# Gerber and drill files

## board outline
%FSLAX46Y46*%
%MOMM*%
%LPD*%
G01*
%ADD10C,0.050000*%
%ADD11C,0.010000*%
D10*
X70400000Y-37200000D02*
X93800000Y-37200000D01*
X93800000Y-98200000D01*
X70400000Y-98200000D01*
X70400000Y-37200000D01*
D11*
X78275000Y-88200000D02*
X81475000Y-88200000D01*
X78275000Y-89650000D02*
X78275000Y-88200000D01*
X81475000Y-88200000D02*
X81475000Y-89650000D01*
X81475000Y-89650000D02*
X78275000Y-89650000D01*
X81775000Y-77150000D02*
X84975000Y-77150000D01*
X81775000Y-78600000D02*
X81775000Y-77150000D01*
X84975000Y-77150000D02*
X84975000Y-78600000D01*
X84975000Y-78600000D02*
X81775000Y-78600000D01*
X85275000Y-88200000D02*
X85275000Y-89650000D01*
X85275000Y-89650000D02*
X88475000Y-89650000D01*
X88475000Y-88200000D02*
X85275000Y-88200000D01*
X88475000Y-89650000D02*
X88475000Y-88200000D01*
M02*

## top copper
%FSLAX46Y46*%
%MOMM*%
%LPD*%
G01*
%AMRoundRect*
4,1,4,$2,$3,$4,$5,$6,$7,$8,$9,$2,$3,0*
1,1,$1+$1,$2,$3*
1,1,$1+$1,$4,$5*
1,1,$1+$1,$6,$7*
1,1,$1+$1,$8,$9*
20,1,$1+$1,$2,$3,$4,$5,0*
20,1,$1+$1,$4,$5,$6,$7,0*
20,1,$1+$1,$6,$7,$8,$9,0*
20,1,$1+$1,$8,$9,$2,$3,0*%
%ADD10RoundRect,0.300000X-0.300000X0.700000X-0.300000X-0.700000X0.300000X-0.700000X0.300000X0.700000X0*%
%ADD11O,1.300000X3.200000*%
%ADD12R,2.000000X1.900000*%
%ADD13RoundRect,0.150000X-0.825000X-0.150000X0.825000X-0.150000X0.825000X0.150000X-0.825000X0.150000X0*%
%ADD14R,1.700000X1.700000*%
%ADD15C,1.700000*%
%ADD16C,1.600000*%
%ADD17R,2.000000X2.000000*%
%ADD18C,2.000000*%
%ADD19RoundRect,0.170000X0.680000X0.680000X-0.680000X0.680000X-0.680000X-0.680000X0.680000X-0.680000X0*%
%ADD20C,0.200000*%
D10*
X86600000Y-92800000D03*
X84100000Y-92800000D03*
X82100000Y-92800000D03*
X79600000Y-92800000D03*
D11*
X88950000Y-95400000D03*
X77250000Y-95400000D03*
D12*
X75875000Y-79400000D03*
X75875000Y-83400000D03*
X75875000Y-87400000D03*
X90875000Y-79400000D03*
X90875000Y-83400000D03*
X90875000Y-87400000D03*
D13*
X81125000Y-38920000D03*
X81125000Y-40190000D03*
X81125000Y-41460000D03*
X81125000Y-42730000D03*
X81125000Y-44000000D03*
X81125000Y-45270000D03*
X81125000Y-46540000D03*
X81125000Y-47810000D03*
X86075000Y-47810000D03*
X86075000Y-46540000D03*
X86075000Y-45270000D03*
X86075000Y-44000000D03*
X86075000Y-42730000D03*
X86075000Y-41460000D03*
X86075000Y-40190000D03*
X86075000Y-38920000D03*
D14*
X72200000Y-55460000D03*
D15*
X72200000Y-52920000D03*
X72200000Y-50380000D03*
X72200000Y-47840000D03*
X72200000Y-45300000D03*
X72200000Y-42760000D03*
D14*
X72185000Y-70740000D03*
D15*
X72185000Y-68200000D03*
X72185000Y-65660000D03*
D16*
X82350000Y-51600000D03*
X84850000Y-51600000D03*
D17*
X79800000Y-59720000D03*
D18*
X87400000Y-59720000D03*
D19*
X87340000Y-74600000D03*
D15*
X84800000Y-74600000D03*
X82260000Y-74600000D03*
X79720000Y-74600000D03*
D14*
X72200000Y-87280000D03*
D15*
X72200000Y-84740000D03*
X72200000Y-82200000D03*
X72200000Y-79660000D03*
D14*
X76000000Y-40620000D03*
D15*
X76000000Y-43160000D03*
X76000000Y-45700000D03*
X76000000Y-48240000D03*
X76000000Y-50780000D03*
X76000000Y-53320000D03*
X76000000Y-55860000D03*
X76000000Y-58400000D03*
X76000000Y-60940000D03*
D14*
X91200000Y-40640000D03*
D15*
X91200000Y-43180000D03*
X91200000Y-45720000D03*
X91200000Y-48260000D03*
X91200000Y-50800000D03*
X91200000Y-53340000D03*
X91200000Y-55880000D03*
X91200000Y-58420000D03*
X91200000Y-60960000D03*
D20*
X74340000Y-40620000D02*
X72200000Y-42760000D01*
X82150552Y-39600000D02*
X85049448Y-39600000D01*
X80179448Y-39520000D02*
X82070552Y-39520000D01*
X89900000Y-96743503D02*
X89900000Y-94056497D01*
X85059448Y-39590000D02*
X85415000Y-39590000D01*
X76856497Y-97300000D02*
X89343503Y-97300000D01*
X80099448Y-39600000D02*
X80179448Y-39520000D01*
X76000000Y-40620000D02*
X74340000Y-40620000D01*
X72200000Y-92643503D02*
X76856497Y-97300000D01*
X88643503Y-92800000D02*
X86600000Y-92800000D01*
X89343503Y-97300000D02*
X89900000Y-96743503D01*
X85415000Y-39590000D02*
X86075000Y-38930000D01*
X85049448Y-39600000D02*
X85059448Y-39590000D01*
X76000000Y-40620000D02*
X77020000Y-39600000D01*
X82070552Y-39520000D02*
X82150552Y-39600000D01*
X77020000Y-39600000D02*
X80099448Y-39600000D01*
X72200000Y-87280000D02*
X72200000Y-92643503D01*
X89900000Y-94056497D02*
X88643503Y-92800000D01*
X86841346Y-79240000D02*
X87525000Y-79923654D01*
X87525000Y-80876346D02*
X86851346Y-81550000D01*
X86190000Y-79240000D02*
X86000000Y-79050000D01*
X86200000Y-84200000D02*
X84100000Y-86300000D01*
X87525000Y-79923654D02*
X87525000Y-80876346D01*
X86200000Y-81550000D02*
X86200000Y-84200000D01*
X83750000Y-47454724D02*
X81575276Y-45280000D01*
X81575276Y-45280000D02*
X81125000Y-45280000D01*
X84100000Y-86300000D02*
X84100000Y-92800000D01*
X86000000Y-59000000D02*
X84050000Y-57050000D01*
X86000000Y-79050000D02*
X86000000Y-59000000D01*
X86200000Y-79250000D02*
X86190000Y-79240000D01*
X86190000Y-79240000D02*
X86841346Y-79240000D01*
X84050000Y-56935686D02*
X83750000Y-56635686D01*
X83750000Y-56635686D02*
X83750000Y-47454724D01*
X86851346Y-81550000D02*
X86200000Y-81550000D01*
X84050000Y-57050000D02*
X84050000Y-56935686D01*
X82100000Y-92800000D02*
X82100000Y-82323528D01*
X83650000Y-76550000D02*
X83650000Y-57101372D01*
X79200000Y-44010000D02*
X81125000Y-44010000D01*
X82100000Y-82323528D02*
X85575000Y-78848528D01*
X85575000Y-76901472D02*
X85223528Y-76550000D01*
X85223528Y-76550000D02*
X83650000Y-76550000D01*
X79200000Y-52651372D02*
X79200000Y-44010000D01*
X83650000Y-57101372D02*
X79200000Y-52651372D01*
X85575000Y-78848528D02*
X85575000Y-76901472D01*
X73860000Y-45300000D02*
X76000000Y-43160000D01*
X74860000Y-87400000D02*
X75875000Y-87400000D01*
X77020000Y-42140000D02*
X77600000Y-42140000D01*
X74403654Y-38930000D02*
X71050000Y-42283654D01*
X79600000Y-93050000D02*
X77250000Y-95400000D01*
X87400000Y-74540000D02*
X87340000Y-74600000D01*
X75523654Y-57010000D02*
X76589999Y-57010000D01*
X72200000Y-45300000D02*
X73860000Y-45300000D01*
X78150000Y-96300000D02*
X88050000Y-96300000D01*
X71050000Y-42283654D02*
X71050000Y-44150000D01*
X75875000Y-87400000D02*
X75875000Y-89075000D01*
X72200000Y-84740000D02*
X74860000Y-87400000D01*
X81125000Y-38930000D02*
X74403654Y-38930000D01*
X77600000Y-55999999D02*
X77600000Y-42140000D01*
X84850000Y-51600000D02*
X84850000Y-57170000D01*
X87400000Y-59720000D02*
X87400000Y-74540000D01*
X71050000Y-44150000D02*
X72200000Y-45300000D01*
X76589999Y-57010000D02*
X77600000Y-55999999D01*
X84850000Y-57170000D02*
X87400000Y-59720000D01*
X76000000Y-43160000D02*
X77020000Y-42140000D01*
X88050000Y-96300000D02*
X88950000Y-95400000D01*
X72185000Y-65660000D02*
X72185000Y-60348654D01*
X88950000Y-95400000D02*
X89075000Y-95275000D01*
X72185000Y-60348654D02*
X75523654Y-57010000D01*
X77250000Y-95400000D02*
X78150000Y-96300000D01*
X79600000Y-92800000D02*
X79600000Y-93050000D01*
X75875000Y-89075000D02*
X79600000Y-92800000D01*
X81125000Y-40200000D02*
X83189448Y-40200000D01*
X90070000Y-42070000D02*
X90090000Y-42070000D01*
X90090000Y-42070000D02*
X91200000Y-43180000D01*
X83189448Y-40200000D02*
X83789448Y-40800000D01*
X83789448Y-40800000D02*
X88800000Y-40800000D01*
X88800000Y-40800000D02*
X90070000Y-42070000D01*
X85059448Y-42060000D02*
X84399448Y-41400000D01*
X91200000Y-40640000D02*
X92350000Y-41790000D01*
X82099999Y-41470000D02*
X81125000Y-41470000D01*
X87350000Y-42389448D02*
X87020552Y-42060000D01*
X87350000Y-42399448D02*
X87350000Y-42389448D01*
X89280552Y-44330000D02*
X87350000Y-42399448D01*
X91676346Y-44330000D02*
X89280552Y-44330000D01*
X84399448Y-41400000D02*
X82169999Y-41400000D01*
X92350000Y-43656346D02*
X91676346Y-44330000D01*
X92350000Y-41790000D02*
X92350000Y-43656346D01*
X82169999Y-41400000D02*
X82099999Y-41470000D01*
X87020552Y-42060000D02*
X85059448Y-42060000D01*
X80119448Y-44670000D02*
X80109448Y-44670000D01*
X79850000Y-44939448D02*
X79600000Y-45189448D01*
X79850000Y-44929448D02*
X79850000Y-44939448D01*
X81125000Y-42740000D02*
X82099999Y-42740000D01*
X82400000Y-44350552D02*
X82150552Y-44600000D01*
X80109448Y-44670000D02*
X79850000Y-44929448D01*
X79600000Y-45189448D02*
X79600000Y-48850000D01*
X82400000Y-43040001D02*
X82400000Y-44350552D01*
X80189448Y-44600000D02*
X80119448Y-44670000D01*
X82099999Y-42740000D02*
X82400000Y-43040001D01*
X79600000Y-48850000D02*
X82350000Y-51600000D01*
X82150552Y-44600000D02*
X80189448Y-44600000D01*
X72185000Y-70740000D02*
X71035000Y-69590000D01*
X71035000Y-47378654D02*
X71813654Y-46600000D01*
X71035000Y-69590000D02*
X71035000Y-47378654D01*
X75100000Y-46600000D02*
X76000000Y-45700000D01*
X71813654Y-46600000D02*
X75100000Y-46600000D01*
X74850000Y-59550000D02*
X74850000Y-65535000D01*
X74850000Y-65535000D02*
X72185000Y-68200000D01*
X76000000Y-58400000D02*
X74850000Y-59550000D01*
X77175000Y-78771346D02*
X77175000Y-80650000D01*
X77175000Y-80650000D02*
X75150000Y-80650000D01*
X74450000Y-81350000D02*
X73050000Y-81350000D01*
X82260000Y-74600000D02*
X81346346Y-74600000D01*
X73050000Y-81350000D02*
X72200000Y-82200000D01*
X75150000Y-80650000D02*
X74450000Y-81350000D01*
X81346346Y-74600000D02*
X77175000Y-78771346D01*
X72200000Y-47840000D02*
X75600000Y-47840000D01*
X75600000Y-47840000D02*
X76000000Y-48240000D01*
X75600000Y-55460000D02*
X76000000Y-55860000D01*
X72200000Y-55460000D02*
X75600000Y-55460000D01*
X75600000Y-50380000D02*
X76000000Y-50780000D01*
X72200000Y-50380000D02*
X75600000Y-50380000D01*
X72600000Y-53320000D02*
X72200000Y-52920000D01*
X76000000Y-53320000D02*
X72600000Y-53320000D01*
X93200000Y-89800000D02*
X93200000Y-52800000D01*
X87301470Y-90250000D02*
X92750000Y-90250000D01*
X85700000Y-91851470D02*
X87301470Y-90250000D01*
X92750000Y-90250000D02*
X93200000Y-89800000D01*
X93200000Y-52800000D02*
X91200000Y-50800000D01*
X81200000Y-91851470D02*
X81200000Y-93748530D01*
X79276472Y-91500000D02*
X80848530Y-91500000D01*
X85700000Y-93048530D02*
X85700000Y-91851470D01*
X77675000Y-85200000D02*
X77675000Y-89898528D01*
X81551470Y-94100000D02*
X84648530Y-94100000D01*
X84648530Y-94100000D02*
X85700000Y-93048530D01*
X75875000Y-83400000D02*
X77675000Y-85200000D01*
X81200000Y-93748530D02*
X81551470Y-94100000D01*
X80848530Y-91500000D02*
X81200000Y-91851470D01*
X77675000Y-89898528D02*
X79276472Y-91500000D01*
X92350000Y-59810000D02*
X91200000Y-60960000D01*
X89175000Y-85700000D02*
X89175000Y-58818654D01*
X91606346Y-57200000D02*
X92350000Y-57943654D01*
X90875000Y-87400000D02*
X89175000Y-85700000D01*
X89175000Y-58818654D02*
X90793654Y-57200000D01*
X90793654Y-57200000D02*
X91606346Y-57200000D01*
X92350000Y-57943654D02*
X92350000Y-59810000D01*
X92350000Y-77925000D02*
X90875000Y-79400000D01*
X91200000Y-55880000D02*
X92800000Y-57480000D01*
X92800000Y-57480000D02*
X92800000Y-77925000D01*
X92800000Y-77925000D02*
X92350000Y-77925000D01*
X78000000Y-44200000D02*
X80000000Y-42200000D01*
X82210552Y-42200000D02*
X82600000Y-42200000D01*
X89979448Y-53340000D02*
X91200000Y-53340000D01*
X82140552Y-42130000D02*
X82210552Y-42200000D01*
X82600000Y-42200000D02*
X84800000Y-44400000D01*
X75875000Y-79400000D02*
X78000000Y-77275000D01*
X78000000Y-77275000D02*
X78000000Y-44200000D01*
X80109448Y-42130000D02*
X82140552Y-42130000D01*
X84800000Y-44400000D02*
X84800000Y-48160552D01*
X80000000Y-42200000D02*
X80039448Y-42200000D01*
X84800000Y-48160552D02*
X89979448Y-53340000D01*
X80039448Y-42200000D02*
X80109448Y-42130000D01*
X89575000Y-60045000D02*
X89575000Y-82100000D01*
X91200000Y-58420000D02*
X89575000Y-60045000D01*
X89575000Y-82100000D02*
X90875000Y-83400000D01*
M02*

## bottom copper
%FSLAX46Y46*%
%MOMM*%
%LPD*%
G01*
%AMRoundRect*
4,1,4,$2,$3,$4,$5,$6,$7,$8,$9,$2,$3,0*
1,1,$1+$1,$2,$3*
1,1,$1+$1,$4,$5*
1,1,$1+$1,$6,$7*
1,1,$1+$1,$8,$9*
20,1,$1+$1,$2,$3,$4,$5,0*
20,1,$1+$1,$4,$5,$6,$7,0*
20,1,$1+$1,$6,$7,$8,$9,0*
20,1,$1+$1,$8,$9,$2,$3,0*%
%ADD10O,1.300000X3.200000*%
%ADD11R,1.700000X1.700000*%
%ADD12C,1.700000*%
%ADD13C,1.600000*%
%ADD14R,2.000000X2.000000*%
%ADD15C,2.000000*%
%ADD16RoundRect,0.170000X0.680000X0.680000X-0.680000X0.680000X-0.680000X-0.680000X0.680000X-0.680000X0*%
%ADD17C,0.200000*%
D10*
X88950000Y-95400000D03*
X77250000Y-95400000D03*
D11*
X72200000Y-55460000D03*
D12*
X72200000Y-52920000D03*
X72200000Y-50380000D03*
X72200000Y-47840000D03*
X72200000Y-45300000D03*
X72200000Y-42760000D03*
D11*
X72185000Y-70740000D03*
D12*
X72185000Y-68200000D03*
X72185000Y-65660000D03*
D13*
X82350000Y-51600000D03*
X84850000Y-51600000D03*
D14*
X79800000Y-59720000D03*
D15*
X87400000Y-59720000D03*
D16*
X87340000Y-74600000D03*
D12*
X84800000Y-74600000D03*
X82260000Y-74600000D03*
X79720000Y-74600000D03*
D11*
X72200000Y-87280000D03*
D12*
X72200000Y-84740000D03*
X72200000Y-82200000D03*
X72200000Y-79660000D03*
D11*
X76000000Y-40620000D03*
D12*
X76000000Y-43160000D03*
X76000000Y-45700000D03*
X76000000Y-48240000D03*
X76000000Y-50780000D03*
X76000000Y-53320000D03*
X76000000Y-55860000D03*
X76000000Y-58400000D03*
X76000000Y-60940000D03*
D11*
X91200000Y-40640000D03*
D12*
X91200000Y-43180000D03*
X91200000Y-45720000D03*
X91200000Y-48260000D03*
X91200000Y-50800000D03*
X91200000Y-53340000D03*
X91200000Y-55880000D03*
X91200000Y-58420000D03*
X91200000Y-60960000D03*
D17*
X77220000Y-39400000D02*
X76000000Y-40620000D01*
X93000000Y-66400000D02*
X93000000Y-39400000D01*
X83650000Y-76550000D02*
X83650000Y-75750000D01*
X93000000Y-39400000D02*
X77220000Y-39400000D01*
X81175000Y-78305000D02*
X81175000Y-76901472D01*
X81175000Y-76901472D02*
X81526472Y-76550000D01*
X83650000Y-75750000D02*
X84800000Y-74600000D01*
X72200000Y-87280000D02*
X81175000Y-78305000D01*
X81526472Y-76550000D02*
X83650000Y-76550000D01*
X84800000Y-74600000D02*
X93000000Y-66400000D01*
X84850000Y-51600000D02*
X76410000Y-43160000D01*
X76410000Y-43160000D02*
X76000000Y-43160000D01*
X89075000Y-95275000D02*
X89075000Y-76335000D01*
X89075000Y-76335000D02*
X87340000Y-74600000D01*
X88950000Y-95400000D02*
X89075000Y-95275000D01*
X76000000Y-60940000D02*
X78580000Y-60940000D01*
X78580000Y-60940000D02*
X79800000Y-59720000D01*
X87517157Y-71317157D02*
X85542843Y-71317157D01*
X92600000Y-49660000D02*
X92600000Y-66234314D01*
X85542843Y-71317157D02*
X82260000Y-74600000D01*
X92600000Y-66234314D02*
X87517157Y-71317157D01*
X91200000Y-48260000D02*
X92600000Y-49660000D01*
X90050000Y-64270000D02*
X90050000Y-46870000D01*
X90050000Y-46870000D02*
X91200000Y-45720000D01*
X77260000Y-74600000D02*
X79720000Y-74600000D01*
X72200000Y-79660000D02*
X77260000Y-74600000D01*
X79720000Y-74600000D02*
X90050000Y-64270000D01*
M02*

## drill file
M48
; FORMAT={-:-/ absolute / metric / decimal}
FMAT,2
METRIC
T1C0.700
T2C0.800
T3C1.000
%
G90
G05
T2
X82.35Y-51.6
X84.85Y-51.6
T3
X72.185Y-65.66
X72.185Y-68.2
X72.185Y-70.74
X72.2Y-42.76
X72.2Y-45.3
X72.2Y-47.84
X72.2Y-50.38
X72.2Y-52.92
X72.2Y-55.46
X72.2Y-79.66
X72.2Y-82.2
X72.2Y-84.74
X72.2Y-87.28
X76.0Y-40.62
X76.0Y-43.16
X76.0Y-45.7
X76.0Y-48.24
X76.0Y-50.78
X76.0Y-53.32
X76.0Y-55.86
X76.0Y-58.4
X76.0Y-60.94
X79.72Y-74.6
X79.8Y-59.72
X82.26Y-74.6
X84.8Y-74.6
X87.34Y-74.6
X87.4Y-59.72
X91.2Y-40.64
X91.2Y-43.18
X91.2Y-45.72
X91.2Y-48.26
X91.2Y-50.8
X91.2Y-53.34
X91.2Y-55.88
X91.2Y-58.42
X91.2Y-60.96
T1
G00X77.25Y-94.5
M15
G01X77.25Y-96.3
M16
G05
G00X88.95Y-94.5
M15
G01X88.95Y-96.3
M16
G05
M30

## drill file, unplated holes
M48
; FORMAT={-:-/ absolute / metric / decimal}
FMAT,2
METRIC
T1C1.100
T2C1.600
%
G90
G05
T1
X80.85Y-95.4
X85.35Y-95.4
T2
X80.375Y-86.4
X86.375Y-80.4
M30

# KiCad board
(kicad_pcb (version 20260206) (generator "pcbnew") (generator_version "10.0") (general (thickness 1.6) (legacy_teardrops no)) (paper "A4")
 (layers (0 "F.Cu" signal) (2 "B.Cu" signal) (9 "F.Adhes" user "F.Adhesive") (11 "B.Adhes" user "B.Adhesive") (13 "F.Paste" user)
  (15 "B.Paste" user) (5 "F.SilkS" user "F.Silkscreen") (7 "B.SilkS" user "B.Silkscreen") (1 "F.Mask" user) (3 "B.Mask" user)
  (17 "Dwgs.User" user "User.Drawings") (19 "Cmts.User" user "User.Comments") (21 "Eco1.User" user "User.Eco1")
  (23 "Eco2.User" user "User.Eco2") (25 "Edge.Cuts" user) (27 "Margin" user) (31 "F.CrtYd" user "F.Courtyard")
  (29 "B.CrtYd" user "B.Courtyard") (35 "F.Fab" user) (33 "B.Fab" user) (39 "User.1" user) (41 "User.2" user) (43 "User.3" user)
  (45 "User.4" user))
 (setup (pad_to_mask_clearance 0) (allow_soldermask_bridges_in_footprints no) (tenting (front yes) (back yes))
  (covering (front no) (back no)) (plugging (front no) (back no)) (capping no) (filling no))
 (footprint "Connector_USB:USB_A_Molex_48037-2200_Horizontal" (layer "F.Cu") (at 83.1 103.775 -90)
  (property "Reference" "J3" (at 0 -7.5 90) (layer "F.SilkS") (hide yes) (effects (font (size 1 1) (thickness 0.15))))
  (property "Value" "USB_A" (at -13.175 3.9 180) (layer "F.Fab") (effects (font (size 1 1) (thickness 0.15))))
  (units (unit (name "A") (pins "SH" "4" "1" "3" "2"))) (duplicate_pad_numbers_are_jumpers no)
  (pad "" np_thru_hole circle (at -8.375 -2.25 270) (size 1.1 1.1) (drill 1.1) (layers "*.Mask"))
  (pad "" np_thru_hole circle (at -8.375 2.25 270) (size 1.1 1.1) (drill 1.1) (layers "*.Mask"))
  (pad "1" smd roundrect (at -10.975 -3.5 270) (size 2 1.2) (layers "F.Cu" "F.Mask" "F.Paste") (roundrect_rratio 0.25) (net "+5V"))
  (pad "2" smd roundrect (at -10.975 -1 270) (size 2 1.2) (layers "F.Cu" "F.Mask" "F.Paste") (roundrect_rratio 0.25) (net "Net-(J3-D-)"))
  (pad "3" smd roundrect (at -10.975 1 270) (size 2 1.2) (layers "F.Cu" "F.Mask" "F.Paste") (roundrect_rratio 0.25) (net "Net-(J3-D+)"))
  (pad "4" smd roundrect (at -10.975 3.5 270) (size 2 1.2) (layers "F.Cu" "F.Mask" "F.Paste") (roundrect_rratio 0.25) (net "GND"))
  (pad "SH" thru_hole oval (at -8.375 -5.85 270) (size 3.2 1.3) (drill oval 2.5 0.7) (layers "*.Cu" "*.Mask") (remove_unused_layers no)
   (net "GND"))
  (pad "SH" thru_hole oval (at -8.375 5.85 270) (size 3.2 1.3) (drill oval 2.5 0.7) (layers "*.Cu" "*.Mask") (remove_unused_layers no)
   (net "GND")))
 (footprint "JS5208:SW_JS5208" (layer "F.Cu") (at 83.375 83.4)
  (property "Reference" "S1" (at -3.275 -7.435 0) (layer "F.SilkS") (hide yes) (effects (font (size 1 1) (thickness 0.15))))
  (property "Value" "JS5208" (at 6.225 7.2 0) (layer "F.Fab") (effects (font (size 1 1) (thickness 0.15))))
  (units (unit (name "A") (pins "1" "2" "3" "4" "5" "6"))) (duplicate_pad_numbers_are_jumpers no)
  (fp_line (start -5.1 4.8) (end -1.9 4.8) (stroke (width 0.01) (type solid)) (layer "Edge.Cuts"))
  (fp_line (start -5.1 6.25) (end -5.1 4.8) (stroke (width 0.01) (type solid)) (layer "Edge.Cuts"))
  (fp_line (start -1.9 4.8) (end -1.9 6.25) (stroke (width 0.01) (type solid)) (layer "Edge.Cuts"))
  (fp_line (start -1.9 6.25) (end -5.1 6.25) (stroke (width 0.01) (type solid)) (layer "Edge.Cuts"))
  (fp_line (start -1.6 -6.25) (end 1.6 -6.25) (stroke (width 0.01) (type solid)) (layer "Edge.Cuts"))
  (fp_line (start -1.6 -4.8) (end -1.6 -6.25) (stroke (width 0.01) (type solid)) (layer "Edge.Cuts"))
  (fp_line (start 1.6 -6.25) (end 1.6 -4.8) (stroke (width 0.01) (type solid)) (layer "Edge.Cuts"))
  (fp_line (start 1.6 -4.8) (end -1.6 -4.8) (stroke (width 0.01) (type solid)) (layer "Edge.Cuts"))
  (fp_line (start 1.9 4.8) (end 1.9 6.25) (stroke (width 0.01) (type solid)) (layer "Edge.Cuts"))
  (fp_line (start 1.9 6.25) (end 5.1 6.25) (stroke (width 0.01) (type solid)) (layer "Edge.Cuts"))
  (fp_line (start 5.1 4.8) (end 1.9 4.8) (stroke (width 0.01) (type solid)) (layer "Edge.Cuts"))
  (fp_line (start 5.1 6.25) (end 5.1 4.8) (stroke (width 0.01) (type solid)) (layer "Edge.Cuts"))
  (pad "" np_thru_hole circle (at -3 3) (size 1.6 1.6) (drill 1.6) (layers "*.Cu" "*.Mask"))
  (pad "" np_thru_hole circle (at 3 -3) (size 1.6 1.6) (drill 1.6) (layers "*.Cu" "*.Mask"))
  (pad "1" smd rect (at -7.5 -4) (size 2 1.9) (layers "F.Cu" "F.Mask" "F.Paste") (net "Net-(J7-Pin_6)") (solder_mask_margin 0.102))
  (pad "2" smd rect (at -7.5 0) (size 2 1.9) (layers "F.Cu" "F.Mask" "F.Paste") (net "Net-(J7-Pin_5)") (solder_mask_margin 0.102))
  (pad "3" smd rect (at -7.5 4) (size 2 1.9) (layers "F.Cu" "F.Mask" "F.Paste") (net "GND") (solder_mask_margin 0.102))
  (pad "4" smd rect (at 7.5 -4) (size 2 1.9) (layers "F.Cu" "F.Mask" "F.Paste") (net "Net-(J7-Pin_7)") (solder_mask_margin 0.102))
  (pad "5" smd rect (at 7.5 0) (size 2 1.9) (layers "F.Cu" "F.Mask" "F.Paste") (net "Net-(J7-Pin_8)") (solder_mask_margin 0.102))
  (pad "6" smd rect (at 7.5 4) (size 2 1.9) (layers "F.Cu" "F.Mask" "F.Paste") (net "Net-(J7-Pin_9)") (solder_mask_margin 0.102)))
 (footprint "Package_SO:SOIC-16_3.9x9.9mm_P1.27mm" (layer "F.Cu") (at 83.6 43.365)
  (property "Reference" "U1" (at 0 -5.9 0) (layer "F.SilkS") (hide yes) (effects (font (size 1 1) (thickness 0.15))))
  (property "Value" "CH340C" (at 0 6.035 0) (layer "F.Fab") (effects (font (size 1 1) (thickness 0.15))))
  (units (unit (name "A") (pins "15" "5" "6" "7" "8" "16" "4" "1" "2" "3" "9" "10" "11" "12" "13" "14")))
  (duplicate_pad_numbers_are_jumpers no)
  (pad "1" smd roundrect (at -2.475 -4.445) (size 1.95 0.6) (layers "F.Cu" "F.Mask" "F.Paste") (roundrect_rratio 0.25) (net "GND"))
  (pad "2" smd roundrect (at -2.475 -3.175) (size 1.95 0.6) (layers "F.Cu" "F.Mask" "F.Paste") (roundrect_rratio 0.25)
   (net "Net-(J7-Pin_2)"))
  (pad "3" smd roundrect (at -2.475 -1.905) (size 1.95 0.6) (layers "F.Cu" "F.Mask" "F.Paste") (roundrect_rratio 0.25)
   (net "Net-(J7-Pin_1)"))
  (pad "4" smd roundrect (at -2.475 -0.635) (size 1.95 0.6) (layers "F.Cu" "F.Mask" "F.Paste") (roundrect_rratio 0.25) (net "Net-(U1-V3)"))
  (pad "5" smd roundrect (at -2.475 0.635) (size 1.95 0.6) (layers "F.Cu" "F.Mask" "F.Paste") (roundrect_rratio 0.25) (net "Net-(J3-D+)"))
  (pad "6" smd roundrect (at -2.475 1.905) (size 1.95 0.6) (layers "F.Cu" "F.Mask" "F.Paste") (roundrect_rratio 0.25) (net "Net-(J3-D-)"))
  (pad "7" smd roundrect (at -2.475 3.175) (size 1.95 0.6) (layers "F.Cu" "F.Mask" "F.Paste") (roundrect_rratio 0.25)
   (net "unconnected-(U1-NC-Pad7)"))
  (pad "8" smd roundrect (at -2.475 4.445) (size 1.95 0.6) (layers "F.Cu" "F.Mask" "F.Paste") (roundrect_rratio 0.25)
   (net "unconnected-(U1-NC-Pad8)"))
  (pad "9" smd roundrect (at 2.475 4.445) (size 1.95 0.6) (layers "F.Cu" "F.Mask" "F.Paste") (roundrect_rratio 0.25)
   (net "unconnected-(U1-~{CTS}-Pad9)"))
  (pad "10" smd roundrect (at 2.475 3.175) (size 1.95 0.6) (layers "F.Cu" "F.Mask" "F.Paste") (roundrect_rratio 0.25)
   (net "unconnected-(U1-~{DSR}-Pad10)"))
  (pad "11" smd roundrect (at 2.475 1.905) (size 1.95 0.6) (layers "F.Cu" "F.Mask" "F.Paste") (roundrect_rratio 0.25)
   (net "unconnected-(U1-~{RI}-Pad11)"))
  (pad "12" smd roundrect (at 2.475 0.635) (size 1.95 0.6) (layers "F.Cu" "F.Mask" "F.Paste") (roundrect_rratio 0.25)
   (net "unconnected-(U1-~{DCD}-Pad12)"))
  (pad "13" smd roundrect (at 2.475 -0.635) (size 1.95 0.6) (layers "F.Cu" "F.Mask" "F.Paste") (roundrect_rratio 0.25)
   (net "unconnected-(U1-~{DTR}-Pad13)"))
  (pad "14" smd roundrect (at 2.475 -1.905) (size 1.95 0.6) (layers "F.Cu" "F.Mask" "F.Paste") (roundrect_rratio 0.25)
   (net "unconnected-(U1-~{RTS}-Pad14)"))
  (pad "15" smd roundrect (at 2.475 -3.175) (size 1.95 0.6) (layers "F.Cu" "F.Mask" "F.Paste") (roundrect_rratio 0.25)
   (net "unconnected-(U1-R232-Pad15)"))
  (pad "16" smd roundrect (at 2.475 -4.445) (size 1.95 0.6) (layers "F.Cu" "F.Mask" "F.Paste") (roundrect_rratio 0.25) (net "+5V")))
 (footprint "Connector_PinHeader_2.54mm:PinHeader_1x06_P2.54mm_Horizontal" (layer "F.Cu") (at 72.2 55.46 180)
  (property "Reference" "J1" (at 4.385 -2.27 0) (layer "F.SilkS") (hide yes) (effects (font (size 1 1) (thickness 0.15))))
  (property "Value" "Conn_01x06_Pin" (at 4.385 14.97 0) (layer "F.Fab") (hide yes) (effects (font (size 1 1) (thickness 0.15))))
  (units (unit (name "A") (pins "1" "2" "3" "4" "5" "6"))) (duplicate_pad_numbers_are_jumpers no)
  (pad "1" thru_hole rect (at 0 0 180) (size 1.7 1.7) (drill 1) (layers "*.Cu" "*.Mask") (remove_unused_layers no) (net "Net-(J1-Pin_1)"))
  (pad "2" thru_hole circle (at 0 2.54 180) (size 1.7 1.7) (drill 1) (layers "*.Cu" "*.Mask") (remove_unused_layers no)
   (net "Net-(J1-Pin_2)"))
  (pad "3" thru_hole circle (at 0 5.08 180) (size 1.7 1.7) (drill 1) (layers "*.Cu" "*.Mask") (remove_unused_layers no)
   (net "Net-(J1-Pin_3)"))
  (pad "4" thru_hole circle (at 0 7.62 180) (size 1.7 1.7) (drill 1) (layers "*.Cu" "*.Mask") (remove_unused_layers no)
   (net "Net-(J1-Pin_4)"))
  (pad "5" thru_hole circle (at 0 10.16 180) (size 1.7 1.7) (drill 1) (layers "*.Cu" "*.Mask") (remove_unused_layers no) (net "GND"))
  (pad "6" thru_hole circle (at 0 12.7 180) (size 1.7 1.7) (drill 1) (layers "*.Cu" "*.Mask") (remove_unused_layers no) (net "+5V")))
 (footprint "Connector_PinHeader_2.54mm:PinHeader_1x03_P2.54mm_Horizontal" (layer "F.Cu") (at 72.185 70.74 180)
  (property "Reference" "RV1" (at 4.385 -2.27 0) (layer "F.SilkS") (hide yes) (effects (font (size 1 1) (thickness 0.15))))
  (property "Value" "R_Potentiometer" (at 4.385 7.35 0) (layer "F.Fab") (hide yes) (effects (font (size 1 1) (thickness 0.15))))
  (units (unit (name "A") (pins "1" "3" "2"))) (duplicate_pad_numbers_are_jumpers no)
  (pad "1" thru_hole rect (at 0 0 180) (size 1.7 1.7) (drill 1) (layers "*.Cu" "*.Mask") (remove_unused_layers no) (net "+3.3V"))
  (pad "2" thru_hole circle (at 0 2.54 180) (size 1.7 1.7) (drill 1) (layers "*.Cu" "*.Mask") (remove_unused_layers no) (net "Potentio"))
  (pad "3" thru_hole circle (at 0 5.08 180) (size 1.7 1.7) (drill 1) (layers "*.Cu" "*.Mask") (remove_unused_layers no) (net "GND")))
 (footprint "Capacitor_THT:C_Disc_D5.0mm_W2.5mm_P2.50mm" (layer "F.Cu") (at 82.35 51.6)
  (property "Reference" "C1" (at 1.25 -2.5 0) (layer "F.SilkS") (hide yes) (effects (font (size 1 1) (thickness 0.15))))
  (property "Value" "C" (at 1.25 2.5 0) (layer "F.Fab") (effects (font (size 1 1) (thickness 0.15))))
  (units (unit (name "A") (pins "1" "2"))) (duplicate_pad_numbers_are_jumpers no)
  (pad "1" thru_hole circle (at 0 0) (size 1.6 1.6) (drill 0.8) (layers "*.Cu" "*.Mask") (remove_unused_layers no) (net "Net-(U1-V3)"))
  (pad "2" thru_hole circle (at 2.5 0) (size 1.6 1.6) (drill 0.8) (layers "*.Cu" "*.Mask") (remove_unused_layers no) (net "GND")))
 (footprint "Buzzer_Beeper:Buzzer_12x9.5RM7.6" (layer "F.Cu") (at 79.8 59.72)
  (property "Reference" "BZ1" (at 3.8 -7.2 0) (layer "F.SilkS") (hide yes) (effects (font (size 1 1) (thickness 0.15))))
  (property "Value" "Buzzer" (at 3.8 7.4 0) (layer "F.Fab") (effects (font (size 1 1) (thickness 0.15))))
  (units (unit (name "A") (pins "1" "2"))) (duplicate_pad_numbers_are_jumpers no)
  (pad "1" thru_hole rect (at 0 0) (size 2 2) (drill 1) (layers "*.Cu" "*.Mask") (remove_unused_layers no) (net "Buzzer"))
  (pad "2" thru_hole circle (at 7.6 0) (size 2 2) (drill 1) (layers "*.Cu" "*.Mask") (remove_unused_layers no) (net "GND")))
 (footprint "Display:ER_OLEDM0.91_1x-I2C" (layer "F.Cu") (at 87.34 74.6 180)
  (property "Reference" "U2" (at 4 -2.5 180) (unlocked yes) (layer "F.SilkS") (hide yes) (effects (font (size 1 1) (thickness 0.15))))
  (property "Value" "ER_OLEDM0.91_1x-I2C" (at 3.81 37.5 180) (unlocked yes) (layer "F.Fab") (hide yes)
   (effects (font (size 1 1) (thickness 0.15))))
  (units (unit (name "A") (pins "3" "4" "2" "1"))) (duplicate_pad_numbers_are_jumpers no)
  (pad "1" thru_hole roundrect (at 0 0 180) (size 1.7 1.7) (drill 1) (layers "*.Cu" "*.Mask") (remove_unused_layers no)
   (roundrect_rratio 0.1) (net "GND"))
  (pad "2" thru_hole circle (at 2.54 0 180) (size 1.7 1.7) (drill 1) (layers "*.Cu" "*.Mask") (remove_unused_layers no) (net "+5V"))
  (pad "3" thru_hole circle (at 5.08 0 180) (size 1.7 1.7) (drill 1) (layers "*.Cu" "*.Mask") (remove_unused_layers no) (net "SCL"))
  (pad "4" thru_hole circle (at 7.62 0 180) (size 1.7 1.7) (drill 1) (layers "*.Cu" "*.Mask") (remove_unused_layers no) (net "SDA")))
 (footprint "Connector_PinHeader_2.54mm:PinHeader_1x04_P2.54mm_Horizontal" (layer "F.Cu") (at 72.2 87.28 180)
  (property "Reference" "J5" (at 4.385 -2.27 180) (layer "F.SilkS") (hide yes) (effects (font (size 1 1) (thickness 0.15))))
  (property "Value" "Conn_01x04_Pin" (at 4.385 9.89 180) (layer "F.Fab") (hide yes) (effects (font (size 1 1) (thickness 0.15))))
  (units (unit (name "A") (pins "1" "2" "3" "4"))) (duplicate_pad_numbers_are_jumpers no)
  (pad "1" thru_hole rect (at 0 0 180) (size 1.7 1.7) (drill 1) (layers "*.Cu" "*.Mask") (remove_unused_layers no) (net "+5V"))
  (pad "2" thru_hole circle (at 0 2.54 180) (size 1.7 1.7) (drill 1) (layers "*.Cu" "*.Mask") (remove_unused_layers no) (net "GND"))
  (pad "3" thru_hole circle (at 0 5.08 180) (size 1.7 1.7) (drill 1) (layers "*.Cu" "*.Mask") (remove_unused_layers no) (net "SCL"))
  (pad "4" thru_hole circle (at 0 7.62 180) (size 1.7 1.7) (drill 1) (layers "*.Cu" "*.Mask") (remove_unused_layers no) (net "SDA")))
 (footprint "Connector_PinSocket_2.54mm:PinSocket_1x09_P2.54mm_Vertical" (layer "B.Cu") (at 76 40.62 180)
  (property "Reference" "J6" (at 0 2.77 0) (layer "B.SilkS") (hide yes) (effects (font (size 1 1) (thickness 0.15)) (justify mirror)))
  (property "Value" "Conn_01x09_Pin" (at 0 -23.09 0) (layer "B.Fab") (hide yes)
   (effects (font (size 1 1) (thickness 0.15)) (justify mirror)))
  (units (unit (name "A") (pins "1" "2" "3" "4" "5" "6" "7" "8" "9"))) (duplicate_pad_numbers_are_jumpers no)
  (pad "1" thru_hole rect (at 0 0 180) (size 1.7 1.7) (drill 1) (layers "*.Cu" "*.Mask") (remove_unused_layers no) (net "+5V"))
  (pad "2" thru_hole circle (at 0 -2.54 180) (size 1.7 1.7) (drill 1) (layers "*.Cu" "*.Mask") (remove_unused_layers no) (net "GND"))
  (pad "3" thru_hole circle (at 0 -5.08 180) (size 1.7 1.7) (drill 1) (layers "*.Cu" "*.Mask") (remove_unused_layers no) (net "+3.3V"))
  (pad "4" thru_hole circle (at 0 -7.62 180) (size 1.7 1.7) (drill 1) (layers "*.Cu" "*.Mask") (remove_unused_layers no)
   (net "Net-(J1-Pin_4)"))
  (pad "5" thru_hole circle (at 0 -10.16 180) (size 1.7 1.7) (drill 1) (layers "*.Cu" "*.Mask") (remove_unused_layers no)
   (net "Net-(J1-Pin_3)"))
  (pad "6" thru_hole circle (at 0 -12.7 180) (size 1.7 1.7) (drill 1) (layers "*.Cu" "*.Mask") (remove_unused_layers no)
   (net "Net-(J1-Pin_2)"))
  (pad "7" thru_hole circle (at 0 -15.24 180) (size 1.7 1.7) (drill 1) (layers "*.Cu" "*.Mask") (remove_unused_layers no)
   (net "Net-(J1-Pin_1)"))
  (pad "8" thru_hole circle (at 0 -17.78 180) (size 1.7 1.7) (drill 1) (layers "*.Cu" "*.Mask") (remove_unused_layers no) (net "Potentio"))
  (pad "9" thru_hole circle (at 0 -20.32 180) (size 1.7 1.7) (drill 1) (layers "*.Cu" "*.Mask") (remove_unused_layers no) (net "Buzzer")))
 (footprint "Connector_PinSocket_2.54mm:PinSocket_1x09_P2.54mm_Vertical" (layer "B.Cu") (at 91.2 40.64 180)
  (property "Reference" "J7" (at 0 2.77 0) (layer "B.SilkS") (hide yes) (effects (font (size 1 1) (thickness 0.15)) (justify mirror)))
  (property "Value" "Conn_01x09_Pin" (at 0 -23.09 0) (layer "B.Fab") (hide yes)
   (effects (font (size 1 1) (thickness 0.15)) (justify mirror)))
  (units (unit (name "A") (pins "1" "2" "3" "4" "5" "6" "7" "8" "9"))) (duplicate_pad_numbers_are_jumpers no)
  (pad "1" thru_hole rect (at 0 0 180) (size 1.7 1.7) (drill 1) (layers "*.Cu" "*.Mask") (remove_unused_layers no) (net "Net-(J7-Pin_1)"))
  (pad "2" thru_hole circle (at 0 -2.54 180) (size 1.7 1.7) (drill 1) (layers "*.Cu" "*.Mask") (remove_unused_layers no)
   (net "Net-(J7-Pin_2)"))
  (pad "3" thru_hole circle (at 0 -5.08 180) (size 1.7 1.7) (drill 1) (layers "*.Cu" "*.Mask") (remove_unused_layers no) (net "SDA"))
  (pad "4" thru_hole circle (at 0 -7.62 180) (size 1.7 1.7) (drill 1) (layers "*.Cu" "*.Mask") (remove_unused_layers no) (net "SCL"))
  (pad "5" thru_hole circle (at 0 -10.16 180) (size 1.7 1.7) (drill 1) (layers "*.Cu" "*.Mask") (remove_unused_layers no)
   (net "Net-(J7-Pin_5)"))
  (pad "6" thru_hole circle (at 0 -12.7 180) (size 1.7 1.7) (drill 1) (layers "*.Cu" "*.Mask") (remove_unused_layers no)
   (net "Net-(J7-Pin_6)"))
  (pad "7" thru_hole circle (at 0 -15.24 180) (size 1.7 1.7) (drill 1) (layers "*.Cu" "*.Mask") (remove_unused_layers no)
   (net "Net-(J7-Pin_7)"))
  (pad "8" thru_hole circle (at 0 -17.78 180) (size 1.7 1.7) (drill 1) (layers "*.Cu" "*.Mask") (remove_unused_layers no)
   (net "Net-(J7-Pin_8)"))
  (pad "9" thru_hole circle (at 0 -20.32 180) (size 1.7 1.7) (drill 1) (layers "*.Cu" "*.Mask") (remove_unused_layers no)
   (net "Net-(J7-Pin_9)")))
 (gr_rect (start 70.4 37.2) (end 93.8 98.2) (stroke (width 0.05) (type default)) (fill no) (layer "Edge.Cuts"))
 (segment (start 74.34 40.62) (end 72.2 42.76) (width 0.2) (layer "F.Cu") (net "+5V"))
 (segment (start 82.150552 39.6) (end 85.049448 39.6) (width 0.2) (layer "F.Cu") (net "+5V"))
 (segment (start 80.179448 39.52) (end 82.070552 39.52) (width 0.2) (layer "F.Cu") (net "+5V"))
 (segment (start 89.9 96.743503) (end 89.9 94.056497) (width 0.2) (layer "F.Cu") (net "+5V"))
 (segment (start 85.059448 39.59) (end 85.415 39.59) (width 0.2) (layer "F.Cu") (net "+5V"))
 (segment (start 76.856497 97.3) (end 89.343503 97.3) (width 0.2) (layer "F.Cu") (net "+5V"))
 (segment (start 80.099448 39.6) (end 80.179448 39.52) (width 0.2) (layer "F.Cu") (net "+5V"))
 (segment (start 76 40.62) (end 74.34 40.62) (width 0.2) (layer "F.Cu") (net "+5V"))
 (segment (start 72.2 92.643503) (end 76.856497 97.3) (width 0.2) (layer "F.Cu") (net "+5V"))
 (segment (start 88.643503 92.8) (end 86.6 92.8) (width 0.2) (layer "F.Cu") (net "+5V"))
 (segment (start 89.343503 97.3) (end 89.9 96.743503) (width 0.2) (layer "F.Cu") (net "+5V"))
 (segment (start 85.415 39.59) (end 86.075 38.93) (width 0.2) (layer "F.Cu") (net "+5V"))
 (segment (start 85.049448 39.6) (end 85.059448 39.59) (width 0.2) (layer "F.Cu") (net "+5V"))
 (segment (start 76 40.62) (end 77.02 39.6) (width 0.2) (layer "F.Cu") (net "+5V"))
 (segment (start 82.070552 39.52) (end 82.150552 39.6) (width 0.2) (layer "F.Cu") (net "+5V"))
 (segment (start 77.02 39.6) (end 80.099448 39.6) (width 0.2) (layer "F.Cu") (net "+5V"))
 (segment (start 72.2 87.28) (end 72.2 92.643503) (width 0.2) (layer "F.Cu") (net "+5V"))
 (segment (start 89.9 94.056497) (end 88.643503 92.8) (width 0.2) (layer "F.Cu") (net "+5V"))
 (segment (start 77.22 39.4) (end 76 40.62) (width 0.2) (layer "B.Cu") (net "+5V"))
 (segment (start 93 66.4) (end 93 39.4) (width 0.2) (layer "B.Cu") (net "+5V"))
 (segment (start 83.65 76.55) (end 83.65 75.75) (width 0.2) (layer "B.Cu") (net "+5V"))
 (segment (start 93 39.4) (end 77.22 39.4) (width 0.2) (layer "B.Cu") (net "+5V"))
 (segment (start 81.175 78.305) (end 81.175 76.901472) (width 0.2) (layer "B.Cu") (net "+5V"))
 (segment (start 81.175 76.901472) (end 81.526472 76.55) (width 0.2) (layer "B.Cu") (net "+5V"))
 (segment (start 83.65 75.75) (end 84.8 74.6) (width 0.2) (layer "B.Cu") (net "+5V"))
 (segment (start 72.2 87.28) (end 81.175 78.305) (width 0.2) (layer "B.Cu") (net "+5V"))
 (segment (start 81.526472 76.55) (end 83.65 76.55) (width 0.2) (layer "B.Cu") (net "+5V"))
 (segment (start 84.8 74.6) (end 93 66.4) (width 0.2) (layer "B.Cu") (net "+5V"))
 (segment (start 86.841346 79.24) (end 87.525 79.923654) (width 0.2) (layer "F.Cu") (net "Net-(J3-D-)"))
 (segment (start 87.525 80.876346) (end 86.851346 81.55) (width 0.2) (layer "F.Cu") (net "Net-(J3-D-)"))
 (segment (start 86.19 79.24) (end 86 79.05) (width 0.2) (layer "F.Cu") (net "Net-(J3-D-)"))
 (segment (start 86.2 84.2) (end 84.1 86.3) (width 0.2) (layer "F.Cu") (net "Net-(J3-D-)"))
 (segment (start 87.525 79.923654) (end 87.525 80.876346) (width 0.2) (layer "F.Cu") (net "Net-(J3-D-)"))
 (segment (start 86.2 81.55) (end 86.2 84.2) (width 0.2) (layer "F.Cu") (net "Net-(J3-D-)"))
 (segment (start 83.75 47.454724) (end 81.575276 45.28) (width 0.2) (layer "F.Cu") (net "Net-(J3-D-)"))
 (segment (start 81.575276 45.28) (end 81.125 45.28) (width 0.2) (layer "F.Cu") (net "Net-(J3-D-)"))
 (segment (start 84.1 86.3) (end 84.1 92.8) (width 0.2) (layer "F.Cu") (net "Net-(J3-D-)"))
 (segment (start 86 59) (end 84.05 57.05) (width 0.2) (layer "F.Cu") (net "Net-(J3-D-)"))
 (segment (start 86 79.05) (end 86 59) (width 0.2) (layer "F.Cu") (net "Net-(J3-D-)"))
 (segment (start 86.2 79.25) (end 86.19 79.24) (width 0.2) (layer "F.Cu") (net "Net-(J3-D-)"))
 (segment (start 86.19 79.24) (end 86.841346 79.24) (width 0.2) (layer "F.Cu") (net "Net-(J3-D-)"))
 (segment (start 84.05 56.935686) (end 83.75 56.635686) (width 0.2) (layer "F.Cu") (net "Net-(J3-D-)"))
 (segment (start 83.75 56.635686) (end 83.75 47.454724) (width 0.2) (layer "F.Cu") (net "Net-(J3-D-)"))
 (segment (start 86.851346 81.55) (end 86.2 81.55) (width 0.2) (layer "F.Cu") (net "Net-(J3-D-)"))
 (segment (start 84.05 57.05) (end 84.05 56.935686) (width 0.2) (layer "F.Cu") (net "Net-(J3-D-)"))
 (segment (start 82.1 92.8) (end 82.1 82.323528) (width 0.2) (layer "F.Cu") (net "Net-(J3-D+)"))
 (segment (start 83.65 76.55) (end 83.65 57.101372) (width 0.2) (layer "F.Cu") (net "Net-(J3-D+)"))
 (segment (start 79.2 44.01) (end 81.125 44.01) (width 0.2) (layer "F.Cu") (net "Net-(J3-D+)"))
 (segment (start 82.1 82.323528) (end 85.575 78.848528) (width 0.2) (layer "F.Cu") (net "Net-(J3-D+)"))
 (segment (start 85.575 76.901472) (end 85.223528 76.55) (width 0.2) (layer "F.Cu") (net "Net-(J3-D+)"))
 (segment (start 85.223528 76.55) (end 83.65 76.55) (width 0.2) (layer "F.Cu") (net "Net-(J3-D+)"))
 (segment (start 79.2 52.651372) (end 79.2 44.01) (width 0.2) (layer "F.Cu") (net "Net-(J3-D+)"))
 (segment (start 83.65 57.101372) (end 79.2 52.651372) (width 0.2) (layer "F.Cu") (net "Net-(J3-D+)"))
 (segment (start 85.575 78.848528) (end 85.575 76.901472) (width 0.2) (layer "F.Cu") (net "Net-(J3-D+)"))
 (segment (start 73.86 45.3) (end 76 43.16) (width 0.2) (layer "F.Cu") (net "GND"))
 (segment (start 74.86 87.4) (end 75.875 87.4) (width 0.2) (layer "F.Cu") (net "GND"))
 (segment (start 77.02 42.14) (end 77.6 42.14) (width 0.2) (layer "F.Cu") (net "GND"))
 (segment (start 74.403654 38.93) (end 71.05 42.283654) (width 0.2) (layer "F.Cu") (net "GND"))
 (segment (start 79.6 93.05) (end 77.25 95.4) (width 0.2) (layer "F.Cu") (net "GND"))
 (segment (start 87.4 74.54) (end 87.34 74.6) (width 0.2) (layer "F.Cu") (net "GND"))
 (segment (start 75.523654 57.01) (end 76.589999 57.01) (width 0.2) (layer "F.Cu") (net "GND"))
 (segment (start 72.2 45.3) (end 73.86 45.3) (width 0.2) (layer "F.Cu") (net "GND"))
 (segment (start 78.15 96.3) (end 88.05 96.3) (width 0.2) (layer "F.Cu") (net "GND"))
 (segment (start 71.05 42.283654) (end 71.05 44.15) (width 0.2) (layer "F.Cu") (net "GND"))
 (segment (start 75.875 87.4) (end 75.875 89.075) (width 0.2) (layer "F.Cu") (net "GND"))
 (segment (start 72.2 84.74) (end 74.86 87.4) (width 0.2) (layer "F.Cu") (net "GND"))
 (segment (start 81.125 38.93) (end 74.403654 38.93) (width 0.2) (layer "F.Cu") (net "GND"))
 (segment (start 77.6 55.999999) (end 77.6 42.14) (width 0.2) (layer "F.Cu") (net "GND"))
 (segment (start 84.85 51.6) (end 84.85 57.17) (width 0.2) (layer "F.Cu") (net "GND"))
 (segment (start 87.4 59.72) (end 87.4 74.54) (width 0.2) (layer "F.Cu") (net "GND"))
 (segment (start 71.05 44.15) (end 72.2 45.3) (width 0.2) (layer "F.Cu") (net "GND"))
 (segment (start 76.589999 57.01) (end 77.6 55.999999) (width 0.2) (layer "F.Cu") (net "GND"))
 (segment (start 84.85 57.17) (end 87.4 59.72) (width 0.2) (layer "F.Cu") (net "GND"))
 (segment (start 76 43.16) (end 77.02 42.14) (width 0.2) (layer "F.Cu") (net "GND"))
 (segment (start 88.05 96.3) (end 88.95 95.4) (width 0.2) (layer "F.Cu") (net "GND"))
 (segment (start 72.185 65.66) (end 72.185 60.348654) (width 0.2) (layer "F.Cu") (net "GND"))
 (segment (start 88.95 95.4) (end 89.075 95.275) (width 0.2) (layer "F.Cu") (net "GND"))
 (segment (start 72.185 60.348654) (end 75.523654 57.01) (width 0.2) (layer "F.Cu") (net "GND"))
 (segment (start 77.25 95.4) (end 78.15 96.3) (width 0.2) (layer "F.Cu") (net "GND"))
 (segment (start 79.6 92.8) (end 79.6 93.05) (width 0.2) (layer "F.Cu") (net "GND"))
 (segment (start 75.875 89.075) (end 79.6 92.8) (width 0.2) (layer "F.Cu") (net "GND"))
 (segment (start 84.85 51.6) (end 76.41 43.16) (width 0.2) (layer "B.Cu") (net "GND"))
 (segment (start 76.41 43.16) (end 76 43.16) (width 0.2) (layer "B.Cu") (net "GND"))
 (segment (start 89.075 95.275) (end 89.075 76.335) (width 0.2) (layer "B.Cu") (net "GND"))
 (segment (start 89.075 76.335) (end 87.34 74.6) (width 0.2) (layer "B.Cu") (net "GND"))
 (segment (start 88.95 95.4) (end 89.075 95.275) (width 0.2) (layer "B.Cu") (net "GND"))
 (segment (start 78 44.2) (end 80 42.2) (width 0.2) (layer "F.Cu") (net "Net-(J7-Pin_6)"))
 (segment (start 82.210552 42.2) (end 82.6 42.2) (width 0.2) (layer "F.Cu") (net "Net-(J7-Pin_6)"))
 (segment (start 89.979448 53.34) (end 91.2 53.34) (width 0.2) (layer "F.Cu") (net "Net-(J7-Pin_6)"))
 (segment (start 82.140552 42.13) (end 82.210552 42.2) (width 0.2) (layer "F.Cu") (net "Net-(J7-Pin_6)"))
 (segment (start 82.6 42.2) (end 84.8 44.4) (width 0.2) (layer "F.Cu") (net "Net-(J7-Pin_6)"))
 (segment (start 75.875 79.4) (end 78 77.275) (width 0.2) (layer "F.Cu") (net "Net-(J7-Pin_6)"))
 (segment (start 78 77.275) (end 78 44.2) (width 0.2) (layer "F.Cu") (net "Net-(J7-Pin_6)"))
 (segment (start 80.109448 42.13) (end 82.140552 42.13) (width 0.2) (layer "F.Cu") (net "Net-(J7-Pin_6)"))
 (segment (start 84.8 44.4) (end 84.8 48.160552) (width 0.2) (layer "F.Cu") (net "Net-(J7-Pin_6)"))
 (segment (start 80 42.2) (end 80.039448 42.2) (width 0.2) (layer "F.Cu") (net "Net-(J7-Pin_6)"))
 (segment (start 84.8 48.160552) (end 89.979448 53.34) (width 0.2) (layer "F.Cu") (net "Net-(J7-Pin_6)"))
 (segment (start 80.039448 42.2) (end 80.109448 42.13) (width 0.2) (layer "F.Cu") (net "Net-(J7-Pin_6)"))
 (segment (start 93.2 89.8) (end 93.2 52.8) (width 0.2) (layer "F.Cu") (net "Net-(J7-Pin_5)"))
 (segment (start 87.30147 90.25) (end 92.75 90.25) (width 0.2) (layer "F.Cu") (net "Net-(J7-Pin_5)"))
 (segment (start 85.7 91.85147) (end 87.30147 90.25) (width 0.2) (layer "F.Cu") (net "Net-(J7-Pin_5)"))
 (segment (start 92.75 90.25) (end 93.2 89.8) (width 0.2) (layer "F.Cu") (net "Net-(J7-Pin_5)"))
 (segment (start 93.2 52.8) (end 91.2 50.8) (width 0.2) (layer "F.Cu") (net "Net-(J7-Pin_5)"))
 (segment (start 81.2 91.85147) (end 81.2 93.74853) (width 0.2) (layer "F.Cu") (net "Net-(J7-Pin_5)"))
 (segment (start 79.276472 91.5) (end 80.84853 91.5) (width 0.2) (layer "F.Cu") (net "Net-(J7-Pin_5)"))
 (segment (start 85.7 93.04853) (end 85.7 91.85147) (width 0.2) (layer "F.Cu") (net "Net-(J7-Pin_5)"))
 (segment (start 77.675 85.2) (end 77.675 89.898528) (width 0.2) (layer "F.Cu") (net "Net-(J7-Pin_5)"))
 (segment (start 81.55147 94.1) (end 84.64853 94.1) (width 0.2) (layer "F.Cu") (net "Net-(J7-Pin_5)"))
 (segment (start 84.64853 94.1) (end 85.7 93.04853) (width 0.2) (layer "F.Cu") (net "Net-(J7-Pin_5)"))
 (segment (start 75.875 83.4) (end 77.675 85.2) (width 0.2) (layer "F.Cu") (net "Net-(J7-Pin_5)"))
 (segment (start 81.2 93.74853) (end 81.55147 94.1) (width 0.2) (layer "F.Cu") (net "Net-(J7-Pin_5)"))
 (segment (start 80.84853 91.5) (end 81.2 91.85147) (width 0.2) (layer "F.Cu") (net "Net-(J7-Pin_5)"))
 (segment (start 77.675 89.898528) (end 79.276472 91.5) (width 0.2) (layer "F.Cu") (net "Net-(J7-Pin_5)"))
 (segment (start 92.35 77.925) (end 90.875 79.4) (width 0.2) (layer "F.Cu") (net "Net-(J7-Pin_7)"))
 (segment (start 91.2 55.88) (end 92.8 57.48) (width 0.2) (layer "F.Cu") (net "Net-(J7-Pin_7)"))
 (segment (start 92.8 57.48) (end 92.8 77.925) (width 0.2) (layer "F.Cu") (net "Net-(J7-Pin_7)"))
 (segment (start 92.8 77.925) (end 92.35 77.925) (width 0.2) (layer "F.Cu") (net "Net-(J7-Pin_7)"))
 (segment (start 89.575 60.045) (end 89.575 82.1) (width 0.2) (layer "F.Cu") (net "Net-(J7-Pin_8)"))
 (segment (start 91.2 58.42) (end 89.575 60.045) (width 0.2) (layer "F.Cu") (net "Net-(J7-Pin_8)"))
 (segment (start 89.575 82.1) (end 90.875 83.4) (width 0.2) (layer "F.Cu") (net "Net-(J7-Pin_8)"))
 (segment (start 92.35 59.81) (end 91.2 60.96) (width 0.2) (layer "F.Cu") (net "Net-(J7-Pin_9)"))
 (segment (start 89.175 85.7) (end 89.175 58.818654) (width 0.2) (layer "F.Cu") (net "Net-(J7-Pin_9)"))
 (segment (start 91.606346 57.2) (end 92.35 57.943654) (width 0.2) (layer "F.Cu") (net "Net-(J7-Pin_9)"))
 (segment (start 90.875 87.4) (end 89.175 85.7) (width 0.2) (layer "F.Cu") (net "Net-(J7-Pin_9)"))
 (segment (start 89.175 58.818654) (end 90.793654 57.2) (width 0.2) (layer "F.Cu") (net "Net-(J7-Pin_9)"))
 (segment (start 90.793654 57.2) (end 91.606346 57.2) (width 0.2) (layer "F.Cu") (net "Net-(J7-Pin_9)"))
 (segment (start 92.35 57.943654) (end 92.35 59.81) (width 0.2) (layer "F.Cu") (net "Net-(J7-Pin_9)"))
 (segment (start 81.125 40.2) (end 83.189448 40.2) (width 0.2) (layer "F.Cu") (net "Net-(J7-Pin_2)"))
 (segment (start 90.07 42.07) (end 90.09 42.07) (width 0.2) (layer "F.Cu") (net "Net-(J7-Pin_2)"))
 (segment (start 90.09 42.07) (end 91.2 43.18) (width 0.2) (layer "F.Cu") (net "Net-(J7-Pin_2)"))
 (segment (start 83.189448 40.2) (end 83.789448 40.8) (width 0.2) (layer "F.Cu") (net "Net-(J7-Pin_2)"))
 (segment (start 83.789448 40.8) (end 88.8 40.8) (width 0.2) (layer "F.Cu") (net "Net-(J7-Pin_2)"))
 (segment (start 88.8 40.8) (end 90.07 42.07) (width 0.2) (layer "F.Cu") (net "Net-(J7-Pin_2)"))
 (segment (start 85.059448 42.06) (end 84.399448 41.4) (width 0.2) (layer "F.Cu") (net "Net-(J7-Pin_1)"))
 (segment (start 91.2 40.64) (end 92.35 41.79) (width 0.2) (layer "F.Cu") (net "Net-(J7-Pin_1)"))
 (segment (start 82.099999 41.47) (end 81.125 41.47) (width 0.2) (layer "F.Cu") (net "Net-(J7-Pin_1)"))
 (segment (start 87.35 42.389448) (end 87.020552 42.06) (width 0.2) (layer "F.Cu") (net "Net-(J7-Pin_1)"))
 (segment (start 87.35 42.399448) (end 87.35 42.389448) (width 0.2) (layer "F.Cu") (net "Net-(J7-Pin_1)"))
 (segment (start 89.280552 44.33) (end 87.35 42.399448) (width 0.2) (layer "F.Cu") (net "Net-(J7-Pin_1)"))
 (segment (start 91.676346 44.33) (end 89.280552 44.33) (width 0.2) (layer "F.Cu") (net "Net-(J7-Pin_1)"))
 (segment (start 84.399448 41.4) (end 82.169999 41.4) (width 0.2) (layer "F.Cu") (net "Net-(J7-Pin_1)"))
 (segment (start 92.35 43.656346) (end 91.676346 44.33) (width 0.2) (layer "F.Cu") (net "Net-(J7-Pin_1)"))
 (segment (start 92.35 41.79) (end 92.35 43.656346) (width 0.2) (layer "F.Cu") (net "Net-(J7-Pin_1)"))
 (segment (start 82.169999 41.4) (end 82.099999 41.47) (width 0.2) (layer "F.Cu") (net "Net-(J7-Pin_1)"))
 (segment (start 87.020552 42.06) (end 85.059448 42.06) (width 0.2) (layer "F.Cu") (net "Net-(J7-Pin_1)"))
 (segment (start 80.119448 44.67) (end 80.109448 44.67) (width 0.2) (layer "F.Cu") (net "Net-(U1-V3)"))
 (segment (start 79.85 44.939448) (end 79.6 45.189448) (width 0.2) (layer "F.Cu") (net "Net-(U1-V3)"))
 (segment (start 79.85 44.929448) (end 79.85 44.939448) (width 0.2) (layer "F.Cu") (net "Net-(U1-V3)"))
 (segment (start 81.125 42.74) (end 82.099999 42.74) (width 0.2) (layer "F.Cu") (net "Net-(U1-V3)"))
 (segment (start 82.4 44.350552) (end 82.150552 44.6) (width 0.2) (layer "F.Cu") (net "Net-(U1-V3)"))
 (segment (start 80.109448 44.67) (end 79.85 44.929448) (width 0.2) (layer "F.Cu") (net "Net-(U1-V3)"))
 (segment (start 79.6 45.189448) (end 79.6 48.85) (width 0.2) (layer "F.Cu") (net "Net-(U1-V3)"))
 (segment (start 82.4 43.040001) (end 82.4 44.350552) (width 0.2) (layer "F.Cu") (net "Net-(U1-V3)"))
 (segment (start 80.189448 44.6) (end 80.119448 44.67) (width 0.2) (layer "F.Cu") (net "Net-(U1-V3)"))
 (segment (start 82.099999 42.74) (end 82.4 43.040001) (width 0.2) (layer "F.Cu") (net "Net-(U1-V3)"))
 (segment (start 79.6 48.85) (end 82.35 51.6) (width 0.2) (layer "F.Cu") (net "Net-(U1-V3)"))
 (segment (start 82.150552 44.6) (end 80.189448 44.6) (width 0.2) (layer "F.Cu") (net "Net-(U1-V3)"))
 (segment (start 75.6 55.46) (end 76 55.86) (width 0.2) (layer "F.Cu") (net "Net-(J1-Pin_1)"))
 (segment (start 72.2 55.46) (end 75.6 55.46) (width 0.2) (layer "F.Cu") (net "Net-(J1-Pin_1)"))
 (segment (start 72.6 53.32) (end 72.2 52.92) (width 0.2) (layer "F.Cu") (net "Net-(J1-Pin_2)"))
 (segment (start 76 53.32) (end 72.6 53.32) (width 0.2) (layer "F.Cu") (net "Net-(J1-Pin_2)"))
 (segment (start 75.6 50.38) (end 76 50.78) (width 0.2) (layer "F.Cu") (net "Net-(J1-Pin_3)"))
 (segment (start 72.2 50.38) (end 75.6 50.38) (width 0.2) (layer "F.Cu") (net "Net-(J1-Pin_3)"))
 (segment (start 72.2 47.84) (end 75.6 47.84) (width 0.2) (layer "F.Cu") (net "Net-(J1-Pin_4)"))
 (segment (start 75.6 47.84) (end 76 48.24) (width 0.2) (layer "F.Cu") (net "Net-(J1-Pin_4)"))
 (segment (start 72.185 70.74) (end 71.035 69.59) (width 0.2) (layer "F.Cu") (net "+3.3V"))
 (segment (start 71.035 47.378654) (end 71.813654 46.6) (width 0.2) (layer "F.Cu") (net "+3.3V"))
 (segment (start 71.035 69.59) (end 71.035 47.378654) (width 0.2) (layer "F.Cu") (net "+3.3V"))
 (segment (start 75.1 46.6) (end 76 45.7) (width 0.2) (layer "F.Cu") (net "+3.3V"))
 (segment (start 71.813654 46.6) (end 75.1 46.6) (width 0.2) (layer "F.Cu") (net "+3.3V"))
 (segment (start 74.85 59.55) (end 74.85 65.535) (width 0.2) (layer "F.Cu") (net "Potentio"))
 (segment (start 74.85 65.535) (end 72.185 68.2) (width 0.2) (layer "F.Cu") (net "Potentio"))
 (segment (start 76 58.4) (end 74.85 59.55) (width 0.2) (layer "F.Cu") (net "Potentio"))
 (segment (start 76 60.94) (end 78.58 60.94) (width 0.2) (layer "B.Cu") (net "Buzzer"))
 (segment (start 78.58 60.94) (end 79.8 59.72) (width 0.2) (layer "B.Cu") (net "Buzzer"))
 (segment (start 77.175 78.771346) (end 77.175 80.65) (width 0.2) (layer "F.Cu") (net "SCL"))
 (segment (start 77.175 80.65) (end 75.15 80.65) (width 0.2) (layer "F.Cu") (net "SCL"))
 (segment (start 74.45 81.35) (end 73.05 81.35) (width 0.2) (layer "F.Cu") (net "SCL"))
 (segment (start 82.26 74.6) (end 81.346346 74.6) (width 0.2) (layer "F.Cu") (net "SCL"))
 (segment (start 73.05 81.35) (end 72.2 82.2) (width 0.2) (layer "F.Cu") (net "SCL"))
 (segment (start 75.15 80.65) (end 74.45 81.35) (width 0.2) (layer "F.Cu") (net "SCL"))
 (segment (start 81.346346 74.6) (end 77.175 78.771346) (width 0.2) (layer "F.Cu") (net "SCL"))
 (segment (start 87.517157 71.317157) (end 85.542843 71.317157) (width 0.2) (layer "B.Cu") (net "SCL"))
 (segment (start 92.6 49.66) (end 92.6 66.234314) (width 0.2) (layer "B.Cu") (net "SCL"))
 (segment (start 85.542843 71.317157) (end 82.26 74.6) (width 0.2) (layer "B.Cu") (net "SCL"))
 (segment (start 92.6 66.234314) (end 87.517157 71.317157) (width 0.2) (layer "B.Cu") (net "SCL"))
 (segment (start 91.2 48.26) (end 92.6 49.66) (width 0.2) (layer "B.Cu") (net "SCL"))
 (segment (start 90.05 64.27) (end 90.05 46.87) (width 0.2) (layer "B.Cu") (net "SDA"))
 (segment (start 90.05 46.87) (end 91.2 45.72) (width 0.2) (layer "B.Cu") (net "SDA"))
 (segment (start 77.26 74.6) (end 79.72 74.6) (width 0.2) (layer "B.Cu") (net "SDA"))
 (segment (start 72.2 79.66) (end 77.26 74.6) (width 0.2) (layer "B.Cu") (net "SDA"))
 (segment (start 79.72 74.6) (end 90.05 64.27) (width 0.2) (layer "B.Cu") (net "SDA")))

